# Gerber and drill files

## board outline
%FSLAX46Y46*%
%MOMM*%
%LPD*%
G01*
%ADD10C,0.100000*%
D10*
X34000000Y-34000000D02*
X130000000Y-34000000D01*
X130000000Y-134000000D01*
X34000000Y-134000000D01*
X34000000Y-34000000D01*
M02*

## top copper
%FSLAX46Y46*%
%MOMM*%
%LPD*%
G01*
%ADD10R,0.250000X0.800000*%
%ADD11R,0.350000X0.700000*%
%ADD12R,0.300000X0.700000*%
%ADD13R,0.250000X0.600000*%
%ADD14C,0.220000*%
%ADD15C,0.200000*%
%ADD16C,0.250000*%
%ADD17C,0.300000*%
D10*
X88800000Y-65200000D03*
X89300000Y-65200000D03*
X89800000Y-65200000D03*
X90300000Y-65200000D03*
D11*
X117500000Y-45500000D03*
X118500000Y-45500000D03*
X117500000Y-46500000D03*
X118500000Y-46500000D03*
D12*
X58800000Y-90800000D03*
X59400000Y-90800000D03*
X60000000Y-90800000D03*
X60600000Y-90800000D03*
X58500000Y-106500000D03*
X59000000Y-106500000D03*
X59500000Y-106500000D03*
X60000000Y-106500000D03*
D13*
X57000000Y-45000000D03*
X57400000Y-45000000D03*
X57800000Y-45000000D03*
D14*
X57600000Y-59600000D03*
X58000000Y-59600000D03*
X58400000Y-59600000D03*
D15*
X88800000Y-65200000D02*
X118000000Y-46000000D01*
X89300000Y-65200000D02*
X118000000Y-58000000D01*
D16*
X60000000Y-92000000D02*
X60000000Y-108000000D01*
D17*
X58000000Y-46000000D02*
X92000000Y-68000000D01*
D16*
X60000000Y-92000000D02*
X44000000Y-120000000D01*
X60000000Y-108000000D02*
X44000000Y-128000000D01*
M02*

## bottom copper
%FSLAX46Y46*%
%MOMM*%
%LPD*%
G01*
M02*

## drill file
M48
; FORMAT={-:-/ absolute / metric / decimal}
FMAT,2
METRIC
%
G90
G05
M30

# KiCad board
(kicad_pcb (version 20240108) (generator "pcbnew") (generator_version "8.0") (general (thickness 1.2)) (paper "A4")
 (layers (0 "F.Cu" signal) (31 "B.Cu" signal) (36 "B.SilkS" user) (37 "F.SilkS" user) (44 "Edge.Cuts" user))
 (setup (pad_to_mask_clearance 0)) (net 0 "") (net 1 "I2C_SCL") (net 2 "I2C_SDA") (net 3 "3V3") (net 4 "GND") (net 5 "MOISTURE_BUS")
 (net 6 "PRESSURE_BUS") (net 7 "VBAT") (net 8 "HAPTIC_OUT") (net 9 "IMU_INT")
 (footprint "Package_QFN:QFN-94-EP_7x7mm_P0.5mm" (layer "F.Cu") (at 92 68)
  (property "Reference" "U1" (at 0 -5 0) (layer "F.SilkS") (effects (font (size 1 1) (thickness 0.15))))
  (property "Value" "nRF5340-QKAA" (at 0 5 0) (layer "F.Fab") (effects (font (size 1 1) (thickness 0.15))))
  (pad "1" smd rect (at -3.2 -2.8) (size 0.25 0.8) (layers "F.Cu" "F.Paste" "F.Mask") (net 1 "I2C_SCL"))
  (pad "2" smd rect (at -2.7 -2.8) (size 0.25 0.8) (layers "F.Cu" "F.Paste" "F.Mask") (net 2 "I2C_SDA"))
  (pad "3" smd rect (at -2.2 -2.8) (size 0.25 0.8) (layers "F.Cu" "F.Paste" "F.Mask") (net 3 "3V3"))
  (pad "4" smd rect (at -1.7 -2.8) (size 0.25 0.8) (layers "F.Cu" "F.Paste" "F.Mask") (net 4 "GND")))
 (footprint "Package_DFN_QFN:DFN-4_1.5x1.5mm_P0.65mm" (layer "F.Cu") (at 118 46)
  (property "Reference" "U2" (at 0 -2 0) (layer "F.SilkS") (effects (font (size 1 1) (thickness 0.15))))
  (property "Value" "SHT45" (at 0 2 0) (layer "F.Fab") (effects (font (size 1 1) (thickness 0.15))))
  (pad "1" smd rect (at -0.5 -0.5) (size 0.35 0.7) (layers "F.Cu" "F.Paste" "F.Mask") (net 1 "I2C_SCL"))
  (pad "2" smd rect (at 0.5 -0.5) (size 0.35 0.7) (layers "F.Cu" "F.Paste" "F.Mask") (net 2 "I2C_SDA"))
  (pad "3" smd rect (at -0.5 0.5) (size 0.35 0.7) (layers "F.Cu" "F.Paste" "F.Mask") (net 3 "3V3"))
  (pad "4" smd rect (at 0.5 0.5) (size 0.35 0.7) (layers "F.Cu" "F.Paste" "F.Mask") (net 4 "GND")))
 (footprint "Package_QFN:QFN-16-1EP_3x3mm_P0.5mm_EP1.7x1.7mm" (layer "F.Cu") (at 60 92)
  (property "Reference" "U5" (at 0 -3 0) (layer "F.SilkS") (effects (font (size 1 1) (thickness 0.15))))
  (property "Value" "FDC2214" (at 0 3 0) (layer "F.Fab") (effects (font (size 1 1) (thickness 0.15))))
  (pad "1" smd rect (at -1.2 -1.2) (size 0.3 0.7) (layers "F.Cu" "F.Paste" "F.Mask") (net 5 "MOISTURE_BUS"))
  (pad "2" smd rect (at -0.6 -1.2) (size 0.3 0.7) (layers "F.Cu" "F.Paste" "F.Mask") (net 1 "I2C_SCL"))
  (pad "3" smd rect (at 0.0 -1.2) (size 0.3 0.7) (layers "F.Cu" "F.Paste" "F.Mask") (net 2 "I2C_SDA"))
  (pad "4" smd rect (at 0.6 -1.2) (size 0.3 0.7) (layers "F.Cu" "F.Paste" "F.Mask") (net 3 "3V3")))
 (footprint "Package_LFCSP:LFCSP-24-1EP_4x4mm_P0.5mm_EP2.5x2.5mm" (layer "F.Cu") (at 60 108)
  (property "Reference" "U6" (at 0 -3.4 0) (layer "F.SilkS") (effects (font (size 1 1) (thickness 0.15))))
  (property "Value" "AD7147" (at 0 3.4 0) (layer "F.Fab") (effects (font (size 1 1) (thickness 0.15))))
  (pad "1" smd rect (at -1.5 -1.5) (size 0.3 0.7) (layers "F.Cu" "F.Paste" "F.Mask") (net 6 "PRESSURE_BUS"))
  (pad "2" smd rect (at -1.0 -1.5) (size 0.3 0.7) (layers "F.Cu" "F.Paste" "F.Mask") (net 1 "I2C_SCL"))
  (pad "3" smd rect (at -0.5 -1.5) (size 0.3 0.7) (layers "F.Cu" "F.Paste" "F.Mask") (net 2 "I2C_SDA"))
  (pad "4" smd rect (at 0.0 -1.5) (size 0.3 0.7) (layers "F.Cu" "F.Paste" "F.Mask") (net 3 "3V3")))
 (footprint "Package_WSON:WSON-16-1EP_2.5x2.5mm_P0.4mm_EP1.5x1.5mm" (layer "F.Cu") (at 58 46)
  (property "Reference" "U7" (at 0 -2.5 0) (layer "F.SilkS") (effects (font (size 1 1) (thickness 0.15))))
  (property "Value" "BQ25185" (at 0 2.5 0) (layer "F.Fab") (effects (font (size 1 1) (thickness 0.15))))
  (pad "1" smd rect (at -1.0 -1.0) (size 0.25 0.6) (layers "F.Cu" "F.Paste" "F.Mask") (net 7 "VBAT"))
  (pad "2" smd rect (at -0.6 -1.0) (size 0.25 0.6) (layers "F.Cu" "F.Paste" "F.Mask") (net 3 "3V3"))
  (pad "3" smd rect (at -0.2 -1.0) (size 0.25 0.6) (layers "F.Cu" "F.Paste" "F.Mask") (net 4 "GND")))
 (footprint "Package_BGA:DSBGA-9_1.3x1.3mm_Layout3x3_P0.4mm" (layer "F.Cu") (at 58 60)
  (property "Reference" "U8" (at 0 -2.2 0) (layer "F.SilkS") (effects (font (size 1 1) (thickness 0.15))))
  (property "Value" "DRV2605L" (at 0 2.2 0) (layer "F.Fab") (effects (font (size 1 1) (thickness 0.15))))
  (pad "A1" smd circle (at -0.4 -0.4) (size 0.22 0.22) (layers "F.Cu" "F.Paste" "F.Mask") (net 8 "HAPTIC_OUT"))
  (pad "A2" smd circle (at 0.0 -0.4) (size 0.22 0.22) (layers "F.Cu" "F.Paste" "F.Mask") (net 1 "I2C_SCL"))
  (pad "A3" smd circle (at 0.4 -0.4) (size 0.22 0.22) (layers "F.Cu" "F.Paste" "F.Mask") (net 2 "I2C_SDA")))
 (segment (start 88.8 65.2) (end 118 46) (width 0.2) (layer "F.Cu") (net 1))
 (segment (start 89.3 65.2) (end 118 58) (width 0.2) (layer "F.Cu") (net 2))
 (segment (start 60 92) (end 60 108) (width 0.25) (layer "F.Cu") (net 3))
 (segment (start 58 46) (end 92 68) (width 0.3) (layer "F.Cu") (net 7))
 (segment (start 60 92) (end 44 120) (width 0.25) (layer "F.Cu") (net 5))
 (segment (start 60 108) (end 44 128) (width 0.25) (layer "F.Cu") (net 6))
 (gr_rect (start 34 34) (end 130 134) (stroke (width 0.1) (type solid)) (fill no) (layer "Edge.Cuts")))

